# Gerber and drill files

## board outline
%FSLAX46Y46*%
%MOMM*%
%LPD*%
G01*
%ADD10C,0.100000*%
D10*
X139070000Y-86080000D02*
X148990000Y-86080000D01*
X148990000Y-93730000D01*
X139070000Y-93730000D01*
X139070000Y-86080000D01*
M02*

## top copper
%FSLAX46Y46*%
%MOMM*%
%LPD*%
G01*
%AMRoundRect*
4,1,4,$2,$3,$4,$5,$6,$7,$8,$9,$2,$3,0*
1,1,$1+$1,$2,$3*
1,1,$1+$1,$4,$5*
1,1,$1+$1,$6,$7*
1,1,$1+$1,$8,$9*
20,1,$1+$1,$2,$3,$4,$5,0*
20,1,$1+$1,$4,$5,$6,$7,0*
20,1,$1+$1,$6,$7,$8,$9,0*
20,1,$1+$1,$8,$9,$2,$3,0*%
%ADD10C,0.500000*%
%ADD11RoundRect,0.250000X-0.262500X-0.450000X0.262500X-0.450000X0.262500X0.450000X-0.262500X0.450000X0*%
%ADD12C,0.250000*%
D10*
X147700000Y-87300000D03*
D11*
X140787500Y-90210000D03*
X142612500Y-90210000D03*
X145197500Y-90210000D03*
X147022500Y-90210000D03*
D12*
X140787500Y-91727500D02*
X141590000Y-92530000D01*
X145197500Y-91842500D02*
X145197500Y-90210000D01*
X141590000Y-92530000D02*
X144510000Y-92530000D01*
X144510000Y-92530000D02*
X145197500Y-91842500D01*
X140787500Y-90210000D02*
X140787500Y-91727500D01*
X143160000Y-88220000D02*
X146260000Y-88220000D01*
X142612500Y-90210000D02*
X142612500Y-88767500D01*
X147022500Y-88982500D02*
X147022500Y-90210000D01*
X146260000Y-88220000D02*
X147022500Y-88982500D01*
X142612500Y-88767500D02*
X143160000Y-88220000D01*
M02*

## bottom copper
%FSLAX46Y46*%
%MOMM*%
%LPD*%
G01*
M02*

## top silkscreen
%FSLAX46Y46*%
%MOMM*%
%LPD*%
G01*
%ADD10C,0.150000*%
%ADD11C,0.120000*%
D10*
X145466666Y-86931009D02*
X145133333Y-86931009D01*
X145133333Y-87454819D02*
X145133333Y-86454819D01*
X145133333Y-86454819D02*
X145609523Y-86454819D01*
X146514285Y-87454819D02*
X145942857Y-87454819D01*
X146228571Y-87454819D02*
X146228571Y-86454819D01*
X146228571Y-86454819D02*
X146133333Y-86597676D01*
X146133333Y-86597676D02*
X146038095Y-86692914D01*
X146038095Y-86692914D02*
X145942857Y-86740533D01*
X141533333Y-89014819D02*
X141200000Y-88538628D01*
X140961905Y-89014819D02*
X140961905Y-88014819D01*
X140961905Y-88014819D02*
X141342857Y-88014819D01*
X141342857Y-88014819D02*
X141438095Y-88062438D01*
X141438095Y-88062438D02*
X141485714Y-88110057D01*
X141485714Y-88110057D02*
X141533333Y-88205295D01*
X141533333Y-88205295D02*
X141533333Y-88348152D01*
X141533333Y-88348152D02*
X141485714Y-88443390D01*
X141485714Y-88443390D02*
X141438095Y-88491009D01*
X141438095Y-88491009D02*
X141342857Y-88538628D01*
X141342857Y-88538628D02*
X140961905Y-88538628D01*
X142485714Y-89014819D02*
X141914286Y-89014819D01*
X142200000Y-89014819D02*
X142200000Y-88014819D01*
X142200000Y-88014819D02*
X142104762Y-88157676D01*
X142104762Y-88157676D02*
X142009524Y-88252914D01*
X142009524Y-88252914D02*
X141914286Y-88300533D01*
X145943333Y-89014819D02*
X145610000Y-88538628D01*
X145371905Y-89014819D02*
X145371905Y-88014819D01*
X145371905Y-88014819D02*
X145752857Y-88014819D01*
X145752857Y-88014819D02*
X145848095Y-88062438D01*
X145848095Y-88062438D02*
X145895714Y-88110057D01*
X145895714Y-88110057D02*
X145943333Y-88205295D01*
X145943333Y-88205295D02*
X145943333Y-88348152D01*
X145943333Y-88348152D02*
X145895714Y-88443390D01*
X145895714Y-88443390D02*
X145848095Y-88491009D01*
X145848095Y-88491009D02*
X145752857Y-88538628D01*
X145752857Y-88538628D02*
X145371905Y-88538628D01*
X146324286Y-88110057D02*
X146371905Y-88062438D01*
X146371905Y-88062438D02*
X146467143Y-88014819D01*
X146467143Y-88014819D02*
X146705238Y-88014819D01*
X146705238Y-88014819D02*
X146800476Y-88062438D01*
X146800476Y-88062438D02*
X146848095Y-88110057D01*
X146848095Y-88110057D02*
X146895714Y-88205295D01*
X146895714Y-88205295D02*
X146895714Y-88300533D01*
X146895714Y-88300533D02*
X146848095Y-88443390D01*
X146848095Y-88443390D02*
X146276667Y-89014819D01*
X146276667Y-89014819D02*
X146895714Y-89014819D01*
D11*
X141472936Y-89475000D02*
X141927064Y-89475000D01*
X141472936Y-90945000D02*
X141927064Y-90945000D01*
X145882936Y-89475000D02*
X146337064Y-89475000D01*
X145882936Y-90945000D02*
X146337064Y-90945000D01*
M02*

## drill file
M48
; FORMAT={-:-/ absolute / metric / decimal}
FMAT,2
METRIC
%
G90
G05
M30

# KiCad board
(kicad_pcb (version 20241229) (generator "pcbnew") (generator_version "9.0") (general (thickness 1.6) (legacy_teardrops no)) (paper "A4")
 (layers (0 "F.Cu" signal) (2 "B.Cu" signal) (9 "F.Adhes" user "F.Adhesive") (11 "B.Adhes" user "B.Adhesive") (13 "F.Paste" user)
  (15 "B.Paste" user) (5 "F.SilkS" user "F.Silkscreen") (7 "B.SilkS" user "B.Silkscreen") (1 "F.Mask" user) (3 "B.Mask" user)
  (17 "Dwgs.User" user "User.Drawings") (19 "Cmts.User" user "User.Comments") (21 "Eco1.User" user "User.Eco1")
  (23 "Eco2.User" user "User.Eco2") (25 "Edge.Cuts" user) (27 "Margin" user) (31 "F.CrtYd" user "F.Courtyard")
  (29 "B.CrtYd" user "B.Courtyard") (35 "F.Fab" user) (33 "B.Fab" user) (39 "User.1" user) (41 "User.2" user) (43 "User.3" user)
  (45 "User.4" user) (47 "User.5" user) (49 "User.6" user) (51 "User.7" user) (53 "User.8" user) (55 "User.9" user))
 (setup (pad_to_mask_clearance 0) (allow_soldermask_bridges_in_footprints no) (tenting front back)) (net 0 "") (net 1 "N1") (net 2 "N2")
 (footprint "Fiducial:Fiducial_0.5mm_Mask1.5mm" (layer "F.Cu") (at 147.7 87.3)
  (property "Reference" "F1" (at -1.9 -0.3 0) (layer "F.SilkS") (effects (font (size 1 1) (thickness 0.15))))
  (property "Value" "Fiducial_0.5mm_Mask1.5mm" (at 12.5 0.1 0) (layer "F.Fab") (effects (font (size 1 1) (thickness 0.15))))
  (pad "" smd circle (at 0 0) (size 0.5 0.5) (layers "F.Cu" "F.Mask") (solder_mask_margin 0.5) (clearance 0.5)))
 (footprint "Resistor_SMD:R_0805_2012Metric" (layer "F.Cu") (at 141.7 90.21)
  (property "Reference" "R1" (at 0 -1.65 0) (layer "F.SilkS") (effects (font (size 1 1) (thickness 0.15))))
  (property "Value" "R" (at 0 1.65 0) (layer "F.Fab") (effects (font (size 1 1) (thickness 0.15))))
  (fp_line (start -0.227064 -0.735) (end 0.227064 -0.735) (stroke (width 0.12) (type solid)) (layer "F.SilkS"))
  (fp_line (start -0.227064 0.735) (end 0.227064 0.735) (stroke (width 0.12) (type solid)) (layer "F.SilkS"))
  (pad "1" smd roundrect (at -0.9125 0) (size 1.025 1.4) (layers "F.Cu" "F.Mask" "F.Paste") (roundrect_rratio 0.243902) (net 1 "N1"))
  (pad "2" smd roundrect (at 0.9125 0) (size 1.025 1.4) (layers "F.Cu" "F.Mask" "F.Paste") (roundrect_rratio 0.243902) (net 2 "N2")))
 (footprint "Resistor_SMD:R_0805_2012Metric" (layer "F.Cu") (at 146.11 90.21)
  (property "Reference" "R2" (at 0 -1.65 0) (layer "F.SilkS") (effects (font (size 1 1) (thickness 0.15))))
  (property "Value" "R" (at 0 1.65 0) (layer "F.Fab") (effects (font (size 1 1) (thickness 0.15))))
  (fp_line (start -0.227064 -0.735) (end 0.227064 -0.735) (stroke (width 0.12) (type solid)) (layer "F.SilkS"))
  (fp_line (start -0.227064 0.735) (end 0.227064 0.735) (stroke (width 0.12) (type solid)) (layer "F.SilkS"))
  (pad "1" smd roundrect (at -0.9125 0) (size 1.025 1.4) (layers "F.Cu" "F.Mask" "F.Paste") (roundrect_rratio 0.243902) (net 1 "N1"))
  (pad "2" smd roundrect (at 0.9125 0) (size 1.025 1.4) (layers "F.Cu" "F.Mask" "F.Paste") (roundrect_rratio 0.243902) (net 2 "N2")))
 (gr_rect (start 139.07 86.08) (end 148.99 93.73) (stroke (width 0.1) (type solid)) (fill no) (layer "Edge.Cuts"))
 (segment (start 140.7875 91.7275) (end 141.59 92.53) (width 0.25) (layer "F.Cu") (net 1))
 (segment (start 145.1975 91.8425) (end 145.1975 90.21) (width 0.25) (layer "F.Cu") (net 1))
 (segment (start 141.59 92.53) (end 144.51 92.53) (width 0.25) (layer "F.Cu") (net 1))
 (segment (start 144.51 92.53) (end 145.1975 91.8425) (width 0.25) (layer "F.Cu") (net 1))
 (segment (start 140.7875 90.21) (end 140.7875 91.7275) (width 0.25) (layer "F.Cu") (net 1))
 (segment (start 143.16 88.22) (end 146.26 88.22) (width 0.25) (layer "F.Cu") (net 2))
 (segment (start 142.6125 90.21) (end 142.6125 88.7675) (width 0.25) (layer "F.Cu") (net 2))
 (segment (start 147.0225 88.9825) (end 147.0225 90.21) (width 0.25) (layer "F.Cu") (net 2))
 (segment (start 146.26 88.22) (end 147.0225 88.9825) (width 0.25) (layer "F.Cu") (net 2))
 (segment (start 142.6125 88.7675) (end 143.16 88.22) (width 0.25) (layer "F.Cu") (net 2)))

